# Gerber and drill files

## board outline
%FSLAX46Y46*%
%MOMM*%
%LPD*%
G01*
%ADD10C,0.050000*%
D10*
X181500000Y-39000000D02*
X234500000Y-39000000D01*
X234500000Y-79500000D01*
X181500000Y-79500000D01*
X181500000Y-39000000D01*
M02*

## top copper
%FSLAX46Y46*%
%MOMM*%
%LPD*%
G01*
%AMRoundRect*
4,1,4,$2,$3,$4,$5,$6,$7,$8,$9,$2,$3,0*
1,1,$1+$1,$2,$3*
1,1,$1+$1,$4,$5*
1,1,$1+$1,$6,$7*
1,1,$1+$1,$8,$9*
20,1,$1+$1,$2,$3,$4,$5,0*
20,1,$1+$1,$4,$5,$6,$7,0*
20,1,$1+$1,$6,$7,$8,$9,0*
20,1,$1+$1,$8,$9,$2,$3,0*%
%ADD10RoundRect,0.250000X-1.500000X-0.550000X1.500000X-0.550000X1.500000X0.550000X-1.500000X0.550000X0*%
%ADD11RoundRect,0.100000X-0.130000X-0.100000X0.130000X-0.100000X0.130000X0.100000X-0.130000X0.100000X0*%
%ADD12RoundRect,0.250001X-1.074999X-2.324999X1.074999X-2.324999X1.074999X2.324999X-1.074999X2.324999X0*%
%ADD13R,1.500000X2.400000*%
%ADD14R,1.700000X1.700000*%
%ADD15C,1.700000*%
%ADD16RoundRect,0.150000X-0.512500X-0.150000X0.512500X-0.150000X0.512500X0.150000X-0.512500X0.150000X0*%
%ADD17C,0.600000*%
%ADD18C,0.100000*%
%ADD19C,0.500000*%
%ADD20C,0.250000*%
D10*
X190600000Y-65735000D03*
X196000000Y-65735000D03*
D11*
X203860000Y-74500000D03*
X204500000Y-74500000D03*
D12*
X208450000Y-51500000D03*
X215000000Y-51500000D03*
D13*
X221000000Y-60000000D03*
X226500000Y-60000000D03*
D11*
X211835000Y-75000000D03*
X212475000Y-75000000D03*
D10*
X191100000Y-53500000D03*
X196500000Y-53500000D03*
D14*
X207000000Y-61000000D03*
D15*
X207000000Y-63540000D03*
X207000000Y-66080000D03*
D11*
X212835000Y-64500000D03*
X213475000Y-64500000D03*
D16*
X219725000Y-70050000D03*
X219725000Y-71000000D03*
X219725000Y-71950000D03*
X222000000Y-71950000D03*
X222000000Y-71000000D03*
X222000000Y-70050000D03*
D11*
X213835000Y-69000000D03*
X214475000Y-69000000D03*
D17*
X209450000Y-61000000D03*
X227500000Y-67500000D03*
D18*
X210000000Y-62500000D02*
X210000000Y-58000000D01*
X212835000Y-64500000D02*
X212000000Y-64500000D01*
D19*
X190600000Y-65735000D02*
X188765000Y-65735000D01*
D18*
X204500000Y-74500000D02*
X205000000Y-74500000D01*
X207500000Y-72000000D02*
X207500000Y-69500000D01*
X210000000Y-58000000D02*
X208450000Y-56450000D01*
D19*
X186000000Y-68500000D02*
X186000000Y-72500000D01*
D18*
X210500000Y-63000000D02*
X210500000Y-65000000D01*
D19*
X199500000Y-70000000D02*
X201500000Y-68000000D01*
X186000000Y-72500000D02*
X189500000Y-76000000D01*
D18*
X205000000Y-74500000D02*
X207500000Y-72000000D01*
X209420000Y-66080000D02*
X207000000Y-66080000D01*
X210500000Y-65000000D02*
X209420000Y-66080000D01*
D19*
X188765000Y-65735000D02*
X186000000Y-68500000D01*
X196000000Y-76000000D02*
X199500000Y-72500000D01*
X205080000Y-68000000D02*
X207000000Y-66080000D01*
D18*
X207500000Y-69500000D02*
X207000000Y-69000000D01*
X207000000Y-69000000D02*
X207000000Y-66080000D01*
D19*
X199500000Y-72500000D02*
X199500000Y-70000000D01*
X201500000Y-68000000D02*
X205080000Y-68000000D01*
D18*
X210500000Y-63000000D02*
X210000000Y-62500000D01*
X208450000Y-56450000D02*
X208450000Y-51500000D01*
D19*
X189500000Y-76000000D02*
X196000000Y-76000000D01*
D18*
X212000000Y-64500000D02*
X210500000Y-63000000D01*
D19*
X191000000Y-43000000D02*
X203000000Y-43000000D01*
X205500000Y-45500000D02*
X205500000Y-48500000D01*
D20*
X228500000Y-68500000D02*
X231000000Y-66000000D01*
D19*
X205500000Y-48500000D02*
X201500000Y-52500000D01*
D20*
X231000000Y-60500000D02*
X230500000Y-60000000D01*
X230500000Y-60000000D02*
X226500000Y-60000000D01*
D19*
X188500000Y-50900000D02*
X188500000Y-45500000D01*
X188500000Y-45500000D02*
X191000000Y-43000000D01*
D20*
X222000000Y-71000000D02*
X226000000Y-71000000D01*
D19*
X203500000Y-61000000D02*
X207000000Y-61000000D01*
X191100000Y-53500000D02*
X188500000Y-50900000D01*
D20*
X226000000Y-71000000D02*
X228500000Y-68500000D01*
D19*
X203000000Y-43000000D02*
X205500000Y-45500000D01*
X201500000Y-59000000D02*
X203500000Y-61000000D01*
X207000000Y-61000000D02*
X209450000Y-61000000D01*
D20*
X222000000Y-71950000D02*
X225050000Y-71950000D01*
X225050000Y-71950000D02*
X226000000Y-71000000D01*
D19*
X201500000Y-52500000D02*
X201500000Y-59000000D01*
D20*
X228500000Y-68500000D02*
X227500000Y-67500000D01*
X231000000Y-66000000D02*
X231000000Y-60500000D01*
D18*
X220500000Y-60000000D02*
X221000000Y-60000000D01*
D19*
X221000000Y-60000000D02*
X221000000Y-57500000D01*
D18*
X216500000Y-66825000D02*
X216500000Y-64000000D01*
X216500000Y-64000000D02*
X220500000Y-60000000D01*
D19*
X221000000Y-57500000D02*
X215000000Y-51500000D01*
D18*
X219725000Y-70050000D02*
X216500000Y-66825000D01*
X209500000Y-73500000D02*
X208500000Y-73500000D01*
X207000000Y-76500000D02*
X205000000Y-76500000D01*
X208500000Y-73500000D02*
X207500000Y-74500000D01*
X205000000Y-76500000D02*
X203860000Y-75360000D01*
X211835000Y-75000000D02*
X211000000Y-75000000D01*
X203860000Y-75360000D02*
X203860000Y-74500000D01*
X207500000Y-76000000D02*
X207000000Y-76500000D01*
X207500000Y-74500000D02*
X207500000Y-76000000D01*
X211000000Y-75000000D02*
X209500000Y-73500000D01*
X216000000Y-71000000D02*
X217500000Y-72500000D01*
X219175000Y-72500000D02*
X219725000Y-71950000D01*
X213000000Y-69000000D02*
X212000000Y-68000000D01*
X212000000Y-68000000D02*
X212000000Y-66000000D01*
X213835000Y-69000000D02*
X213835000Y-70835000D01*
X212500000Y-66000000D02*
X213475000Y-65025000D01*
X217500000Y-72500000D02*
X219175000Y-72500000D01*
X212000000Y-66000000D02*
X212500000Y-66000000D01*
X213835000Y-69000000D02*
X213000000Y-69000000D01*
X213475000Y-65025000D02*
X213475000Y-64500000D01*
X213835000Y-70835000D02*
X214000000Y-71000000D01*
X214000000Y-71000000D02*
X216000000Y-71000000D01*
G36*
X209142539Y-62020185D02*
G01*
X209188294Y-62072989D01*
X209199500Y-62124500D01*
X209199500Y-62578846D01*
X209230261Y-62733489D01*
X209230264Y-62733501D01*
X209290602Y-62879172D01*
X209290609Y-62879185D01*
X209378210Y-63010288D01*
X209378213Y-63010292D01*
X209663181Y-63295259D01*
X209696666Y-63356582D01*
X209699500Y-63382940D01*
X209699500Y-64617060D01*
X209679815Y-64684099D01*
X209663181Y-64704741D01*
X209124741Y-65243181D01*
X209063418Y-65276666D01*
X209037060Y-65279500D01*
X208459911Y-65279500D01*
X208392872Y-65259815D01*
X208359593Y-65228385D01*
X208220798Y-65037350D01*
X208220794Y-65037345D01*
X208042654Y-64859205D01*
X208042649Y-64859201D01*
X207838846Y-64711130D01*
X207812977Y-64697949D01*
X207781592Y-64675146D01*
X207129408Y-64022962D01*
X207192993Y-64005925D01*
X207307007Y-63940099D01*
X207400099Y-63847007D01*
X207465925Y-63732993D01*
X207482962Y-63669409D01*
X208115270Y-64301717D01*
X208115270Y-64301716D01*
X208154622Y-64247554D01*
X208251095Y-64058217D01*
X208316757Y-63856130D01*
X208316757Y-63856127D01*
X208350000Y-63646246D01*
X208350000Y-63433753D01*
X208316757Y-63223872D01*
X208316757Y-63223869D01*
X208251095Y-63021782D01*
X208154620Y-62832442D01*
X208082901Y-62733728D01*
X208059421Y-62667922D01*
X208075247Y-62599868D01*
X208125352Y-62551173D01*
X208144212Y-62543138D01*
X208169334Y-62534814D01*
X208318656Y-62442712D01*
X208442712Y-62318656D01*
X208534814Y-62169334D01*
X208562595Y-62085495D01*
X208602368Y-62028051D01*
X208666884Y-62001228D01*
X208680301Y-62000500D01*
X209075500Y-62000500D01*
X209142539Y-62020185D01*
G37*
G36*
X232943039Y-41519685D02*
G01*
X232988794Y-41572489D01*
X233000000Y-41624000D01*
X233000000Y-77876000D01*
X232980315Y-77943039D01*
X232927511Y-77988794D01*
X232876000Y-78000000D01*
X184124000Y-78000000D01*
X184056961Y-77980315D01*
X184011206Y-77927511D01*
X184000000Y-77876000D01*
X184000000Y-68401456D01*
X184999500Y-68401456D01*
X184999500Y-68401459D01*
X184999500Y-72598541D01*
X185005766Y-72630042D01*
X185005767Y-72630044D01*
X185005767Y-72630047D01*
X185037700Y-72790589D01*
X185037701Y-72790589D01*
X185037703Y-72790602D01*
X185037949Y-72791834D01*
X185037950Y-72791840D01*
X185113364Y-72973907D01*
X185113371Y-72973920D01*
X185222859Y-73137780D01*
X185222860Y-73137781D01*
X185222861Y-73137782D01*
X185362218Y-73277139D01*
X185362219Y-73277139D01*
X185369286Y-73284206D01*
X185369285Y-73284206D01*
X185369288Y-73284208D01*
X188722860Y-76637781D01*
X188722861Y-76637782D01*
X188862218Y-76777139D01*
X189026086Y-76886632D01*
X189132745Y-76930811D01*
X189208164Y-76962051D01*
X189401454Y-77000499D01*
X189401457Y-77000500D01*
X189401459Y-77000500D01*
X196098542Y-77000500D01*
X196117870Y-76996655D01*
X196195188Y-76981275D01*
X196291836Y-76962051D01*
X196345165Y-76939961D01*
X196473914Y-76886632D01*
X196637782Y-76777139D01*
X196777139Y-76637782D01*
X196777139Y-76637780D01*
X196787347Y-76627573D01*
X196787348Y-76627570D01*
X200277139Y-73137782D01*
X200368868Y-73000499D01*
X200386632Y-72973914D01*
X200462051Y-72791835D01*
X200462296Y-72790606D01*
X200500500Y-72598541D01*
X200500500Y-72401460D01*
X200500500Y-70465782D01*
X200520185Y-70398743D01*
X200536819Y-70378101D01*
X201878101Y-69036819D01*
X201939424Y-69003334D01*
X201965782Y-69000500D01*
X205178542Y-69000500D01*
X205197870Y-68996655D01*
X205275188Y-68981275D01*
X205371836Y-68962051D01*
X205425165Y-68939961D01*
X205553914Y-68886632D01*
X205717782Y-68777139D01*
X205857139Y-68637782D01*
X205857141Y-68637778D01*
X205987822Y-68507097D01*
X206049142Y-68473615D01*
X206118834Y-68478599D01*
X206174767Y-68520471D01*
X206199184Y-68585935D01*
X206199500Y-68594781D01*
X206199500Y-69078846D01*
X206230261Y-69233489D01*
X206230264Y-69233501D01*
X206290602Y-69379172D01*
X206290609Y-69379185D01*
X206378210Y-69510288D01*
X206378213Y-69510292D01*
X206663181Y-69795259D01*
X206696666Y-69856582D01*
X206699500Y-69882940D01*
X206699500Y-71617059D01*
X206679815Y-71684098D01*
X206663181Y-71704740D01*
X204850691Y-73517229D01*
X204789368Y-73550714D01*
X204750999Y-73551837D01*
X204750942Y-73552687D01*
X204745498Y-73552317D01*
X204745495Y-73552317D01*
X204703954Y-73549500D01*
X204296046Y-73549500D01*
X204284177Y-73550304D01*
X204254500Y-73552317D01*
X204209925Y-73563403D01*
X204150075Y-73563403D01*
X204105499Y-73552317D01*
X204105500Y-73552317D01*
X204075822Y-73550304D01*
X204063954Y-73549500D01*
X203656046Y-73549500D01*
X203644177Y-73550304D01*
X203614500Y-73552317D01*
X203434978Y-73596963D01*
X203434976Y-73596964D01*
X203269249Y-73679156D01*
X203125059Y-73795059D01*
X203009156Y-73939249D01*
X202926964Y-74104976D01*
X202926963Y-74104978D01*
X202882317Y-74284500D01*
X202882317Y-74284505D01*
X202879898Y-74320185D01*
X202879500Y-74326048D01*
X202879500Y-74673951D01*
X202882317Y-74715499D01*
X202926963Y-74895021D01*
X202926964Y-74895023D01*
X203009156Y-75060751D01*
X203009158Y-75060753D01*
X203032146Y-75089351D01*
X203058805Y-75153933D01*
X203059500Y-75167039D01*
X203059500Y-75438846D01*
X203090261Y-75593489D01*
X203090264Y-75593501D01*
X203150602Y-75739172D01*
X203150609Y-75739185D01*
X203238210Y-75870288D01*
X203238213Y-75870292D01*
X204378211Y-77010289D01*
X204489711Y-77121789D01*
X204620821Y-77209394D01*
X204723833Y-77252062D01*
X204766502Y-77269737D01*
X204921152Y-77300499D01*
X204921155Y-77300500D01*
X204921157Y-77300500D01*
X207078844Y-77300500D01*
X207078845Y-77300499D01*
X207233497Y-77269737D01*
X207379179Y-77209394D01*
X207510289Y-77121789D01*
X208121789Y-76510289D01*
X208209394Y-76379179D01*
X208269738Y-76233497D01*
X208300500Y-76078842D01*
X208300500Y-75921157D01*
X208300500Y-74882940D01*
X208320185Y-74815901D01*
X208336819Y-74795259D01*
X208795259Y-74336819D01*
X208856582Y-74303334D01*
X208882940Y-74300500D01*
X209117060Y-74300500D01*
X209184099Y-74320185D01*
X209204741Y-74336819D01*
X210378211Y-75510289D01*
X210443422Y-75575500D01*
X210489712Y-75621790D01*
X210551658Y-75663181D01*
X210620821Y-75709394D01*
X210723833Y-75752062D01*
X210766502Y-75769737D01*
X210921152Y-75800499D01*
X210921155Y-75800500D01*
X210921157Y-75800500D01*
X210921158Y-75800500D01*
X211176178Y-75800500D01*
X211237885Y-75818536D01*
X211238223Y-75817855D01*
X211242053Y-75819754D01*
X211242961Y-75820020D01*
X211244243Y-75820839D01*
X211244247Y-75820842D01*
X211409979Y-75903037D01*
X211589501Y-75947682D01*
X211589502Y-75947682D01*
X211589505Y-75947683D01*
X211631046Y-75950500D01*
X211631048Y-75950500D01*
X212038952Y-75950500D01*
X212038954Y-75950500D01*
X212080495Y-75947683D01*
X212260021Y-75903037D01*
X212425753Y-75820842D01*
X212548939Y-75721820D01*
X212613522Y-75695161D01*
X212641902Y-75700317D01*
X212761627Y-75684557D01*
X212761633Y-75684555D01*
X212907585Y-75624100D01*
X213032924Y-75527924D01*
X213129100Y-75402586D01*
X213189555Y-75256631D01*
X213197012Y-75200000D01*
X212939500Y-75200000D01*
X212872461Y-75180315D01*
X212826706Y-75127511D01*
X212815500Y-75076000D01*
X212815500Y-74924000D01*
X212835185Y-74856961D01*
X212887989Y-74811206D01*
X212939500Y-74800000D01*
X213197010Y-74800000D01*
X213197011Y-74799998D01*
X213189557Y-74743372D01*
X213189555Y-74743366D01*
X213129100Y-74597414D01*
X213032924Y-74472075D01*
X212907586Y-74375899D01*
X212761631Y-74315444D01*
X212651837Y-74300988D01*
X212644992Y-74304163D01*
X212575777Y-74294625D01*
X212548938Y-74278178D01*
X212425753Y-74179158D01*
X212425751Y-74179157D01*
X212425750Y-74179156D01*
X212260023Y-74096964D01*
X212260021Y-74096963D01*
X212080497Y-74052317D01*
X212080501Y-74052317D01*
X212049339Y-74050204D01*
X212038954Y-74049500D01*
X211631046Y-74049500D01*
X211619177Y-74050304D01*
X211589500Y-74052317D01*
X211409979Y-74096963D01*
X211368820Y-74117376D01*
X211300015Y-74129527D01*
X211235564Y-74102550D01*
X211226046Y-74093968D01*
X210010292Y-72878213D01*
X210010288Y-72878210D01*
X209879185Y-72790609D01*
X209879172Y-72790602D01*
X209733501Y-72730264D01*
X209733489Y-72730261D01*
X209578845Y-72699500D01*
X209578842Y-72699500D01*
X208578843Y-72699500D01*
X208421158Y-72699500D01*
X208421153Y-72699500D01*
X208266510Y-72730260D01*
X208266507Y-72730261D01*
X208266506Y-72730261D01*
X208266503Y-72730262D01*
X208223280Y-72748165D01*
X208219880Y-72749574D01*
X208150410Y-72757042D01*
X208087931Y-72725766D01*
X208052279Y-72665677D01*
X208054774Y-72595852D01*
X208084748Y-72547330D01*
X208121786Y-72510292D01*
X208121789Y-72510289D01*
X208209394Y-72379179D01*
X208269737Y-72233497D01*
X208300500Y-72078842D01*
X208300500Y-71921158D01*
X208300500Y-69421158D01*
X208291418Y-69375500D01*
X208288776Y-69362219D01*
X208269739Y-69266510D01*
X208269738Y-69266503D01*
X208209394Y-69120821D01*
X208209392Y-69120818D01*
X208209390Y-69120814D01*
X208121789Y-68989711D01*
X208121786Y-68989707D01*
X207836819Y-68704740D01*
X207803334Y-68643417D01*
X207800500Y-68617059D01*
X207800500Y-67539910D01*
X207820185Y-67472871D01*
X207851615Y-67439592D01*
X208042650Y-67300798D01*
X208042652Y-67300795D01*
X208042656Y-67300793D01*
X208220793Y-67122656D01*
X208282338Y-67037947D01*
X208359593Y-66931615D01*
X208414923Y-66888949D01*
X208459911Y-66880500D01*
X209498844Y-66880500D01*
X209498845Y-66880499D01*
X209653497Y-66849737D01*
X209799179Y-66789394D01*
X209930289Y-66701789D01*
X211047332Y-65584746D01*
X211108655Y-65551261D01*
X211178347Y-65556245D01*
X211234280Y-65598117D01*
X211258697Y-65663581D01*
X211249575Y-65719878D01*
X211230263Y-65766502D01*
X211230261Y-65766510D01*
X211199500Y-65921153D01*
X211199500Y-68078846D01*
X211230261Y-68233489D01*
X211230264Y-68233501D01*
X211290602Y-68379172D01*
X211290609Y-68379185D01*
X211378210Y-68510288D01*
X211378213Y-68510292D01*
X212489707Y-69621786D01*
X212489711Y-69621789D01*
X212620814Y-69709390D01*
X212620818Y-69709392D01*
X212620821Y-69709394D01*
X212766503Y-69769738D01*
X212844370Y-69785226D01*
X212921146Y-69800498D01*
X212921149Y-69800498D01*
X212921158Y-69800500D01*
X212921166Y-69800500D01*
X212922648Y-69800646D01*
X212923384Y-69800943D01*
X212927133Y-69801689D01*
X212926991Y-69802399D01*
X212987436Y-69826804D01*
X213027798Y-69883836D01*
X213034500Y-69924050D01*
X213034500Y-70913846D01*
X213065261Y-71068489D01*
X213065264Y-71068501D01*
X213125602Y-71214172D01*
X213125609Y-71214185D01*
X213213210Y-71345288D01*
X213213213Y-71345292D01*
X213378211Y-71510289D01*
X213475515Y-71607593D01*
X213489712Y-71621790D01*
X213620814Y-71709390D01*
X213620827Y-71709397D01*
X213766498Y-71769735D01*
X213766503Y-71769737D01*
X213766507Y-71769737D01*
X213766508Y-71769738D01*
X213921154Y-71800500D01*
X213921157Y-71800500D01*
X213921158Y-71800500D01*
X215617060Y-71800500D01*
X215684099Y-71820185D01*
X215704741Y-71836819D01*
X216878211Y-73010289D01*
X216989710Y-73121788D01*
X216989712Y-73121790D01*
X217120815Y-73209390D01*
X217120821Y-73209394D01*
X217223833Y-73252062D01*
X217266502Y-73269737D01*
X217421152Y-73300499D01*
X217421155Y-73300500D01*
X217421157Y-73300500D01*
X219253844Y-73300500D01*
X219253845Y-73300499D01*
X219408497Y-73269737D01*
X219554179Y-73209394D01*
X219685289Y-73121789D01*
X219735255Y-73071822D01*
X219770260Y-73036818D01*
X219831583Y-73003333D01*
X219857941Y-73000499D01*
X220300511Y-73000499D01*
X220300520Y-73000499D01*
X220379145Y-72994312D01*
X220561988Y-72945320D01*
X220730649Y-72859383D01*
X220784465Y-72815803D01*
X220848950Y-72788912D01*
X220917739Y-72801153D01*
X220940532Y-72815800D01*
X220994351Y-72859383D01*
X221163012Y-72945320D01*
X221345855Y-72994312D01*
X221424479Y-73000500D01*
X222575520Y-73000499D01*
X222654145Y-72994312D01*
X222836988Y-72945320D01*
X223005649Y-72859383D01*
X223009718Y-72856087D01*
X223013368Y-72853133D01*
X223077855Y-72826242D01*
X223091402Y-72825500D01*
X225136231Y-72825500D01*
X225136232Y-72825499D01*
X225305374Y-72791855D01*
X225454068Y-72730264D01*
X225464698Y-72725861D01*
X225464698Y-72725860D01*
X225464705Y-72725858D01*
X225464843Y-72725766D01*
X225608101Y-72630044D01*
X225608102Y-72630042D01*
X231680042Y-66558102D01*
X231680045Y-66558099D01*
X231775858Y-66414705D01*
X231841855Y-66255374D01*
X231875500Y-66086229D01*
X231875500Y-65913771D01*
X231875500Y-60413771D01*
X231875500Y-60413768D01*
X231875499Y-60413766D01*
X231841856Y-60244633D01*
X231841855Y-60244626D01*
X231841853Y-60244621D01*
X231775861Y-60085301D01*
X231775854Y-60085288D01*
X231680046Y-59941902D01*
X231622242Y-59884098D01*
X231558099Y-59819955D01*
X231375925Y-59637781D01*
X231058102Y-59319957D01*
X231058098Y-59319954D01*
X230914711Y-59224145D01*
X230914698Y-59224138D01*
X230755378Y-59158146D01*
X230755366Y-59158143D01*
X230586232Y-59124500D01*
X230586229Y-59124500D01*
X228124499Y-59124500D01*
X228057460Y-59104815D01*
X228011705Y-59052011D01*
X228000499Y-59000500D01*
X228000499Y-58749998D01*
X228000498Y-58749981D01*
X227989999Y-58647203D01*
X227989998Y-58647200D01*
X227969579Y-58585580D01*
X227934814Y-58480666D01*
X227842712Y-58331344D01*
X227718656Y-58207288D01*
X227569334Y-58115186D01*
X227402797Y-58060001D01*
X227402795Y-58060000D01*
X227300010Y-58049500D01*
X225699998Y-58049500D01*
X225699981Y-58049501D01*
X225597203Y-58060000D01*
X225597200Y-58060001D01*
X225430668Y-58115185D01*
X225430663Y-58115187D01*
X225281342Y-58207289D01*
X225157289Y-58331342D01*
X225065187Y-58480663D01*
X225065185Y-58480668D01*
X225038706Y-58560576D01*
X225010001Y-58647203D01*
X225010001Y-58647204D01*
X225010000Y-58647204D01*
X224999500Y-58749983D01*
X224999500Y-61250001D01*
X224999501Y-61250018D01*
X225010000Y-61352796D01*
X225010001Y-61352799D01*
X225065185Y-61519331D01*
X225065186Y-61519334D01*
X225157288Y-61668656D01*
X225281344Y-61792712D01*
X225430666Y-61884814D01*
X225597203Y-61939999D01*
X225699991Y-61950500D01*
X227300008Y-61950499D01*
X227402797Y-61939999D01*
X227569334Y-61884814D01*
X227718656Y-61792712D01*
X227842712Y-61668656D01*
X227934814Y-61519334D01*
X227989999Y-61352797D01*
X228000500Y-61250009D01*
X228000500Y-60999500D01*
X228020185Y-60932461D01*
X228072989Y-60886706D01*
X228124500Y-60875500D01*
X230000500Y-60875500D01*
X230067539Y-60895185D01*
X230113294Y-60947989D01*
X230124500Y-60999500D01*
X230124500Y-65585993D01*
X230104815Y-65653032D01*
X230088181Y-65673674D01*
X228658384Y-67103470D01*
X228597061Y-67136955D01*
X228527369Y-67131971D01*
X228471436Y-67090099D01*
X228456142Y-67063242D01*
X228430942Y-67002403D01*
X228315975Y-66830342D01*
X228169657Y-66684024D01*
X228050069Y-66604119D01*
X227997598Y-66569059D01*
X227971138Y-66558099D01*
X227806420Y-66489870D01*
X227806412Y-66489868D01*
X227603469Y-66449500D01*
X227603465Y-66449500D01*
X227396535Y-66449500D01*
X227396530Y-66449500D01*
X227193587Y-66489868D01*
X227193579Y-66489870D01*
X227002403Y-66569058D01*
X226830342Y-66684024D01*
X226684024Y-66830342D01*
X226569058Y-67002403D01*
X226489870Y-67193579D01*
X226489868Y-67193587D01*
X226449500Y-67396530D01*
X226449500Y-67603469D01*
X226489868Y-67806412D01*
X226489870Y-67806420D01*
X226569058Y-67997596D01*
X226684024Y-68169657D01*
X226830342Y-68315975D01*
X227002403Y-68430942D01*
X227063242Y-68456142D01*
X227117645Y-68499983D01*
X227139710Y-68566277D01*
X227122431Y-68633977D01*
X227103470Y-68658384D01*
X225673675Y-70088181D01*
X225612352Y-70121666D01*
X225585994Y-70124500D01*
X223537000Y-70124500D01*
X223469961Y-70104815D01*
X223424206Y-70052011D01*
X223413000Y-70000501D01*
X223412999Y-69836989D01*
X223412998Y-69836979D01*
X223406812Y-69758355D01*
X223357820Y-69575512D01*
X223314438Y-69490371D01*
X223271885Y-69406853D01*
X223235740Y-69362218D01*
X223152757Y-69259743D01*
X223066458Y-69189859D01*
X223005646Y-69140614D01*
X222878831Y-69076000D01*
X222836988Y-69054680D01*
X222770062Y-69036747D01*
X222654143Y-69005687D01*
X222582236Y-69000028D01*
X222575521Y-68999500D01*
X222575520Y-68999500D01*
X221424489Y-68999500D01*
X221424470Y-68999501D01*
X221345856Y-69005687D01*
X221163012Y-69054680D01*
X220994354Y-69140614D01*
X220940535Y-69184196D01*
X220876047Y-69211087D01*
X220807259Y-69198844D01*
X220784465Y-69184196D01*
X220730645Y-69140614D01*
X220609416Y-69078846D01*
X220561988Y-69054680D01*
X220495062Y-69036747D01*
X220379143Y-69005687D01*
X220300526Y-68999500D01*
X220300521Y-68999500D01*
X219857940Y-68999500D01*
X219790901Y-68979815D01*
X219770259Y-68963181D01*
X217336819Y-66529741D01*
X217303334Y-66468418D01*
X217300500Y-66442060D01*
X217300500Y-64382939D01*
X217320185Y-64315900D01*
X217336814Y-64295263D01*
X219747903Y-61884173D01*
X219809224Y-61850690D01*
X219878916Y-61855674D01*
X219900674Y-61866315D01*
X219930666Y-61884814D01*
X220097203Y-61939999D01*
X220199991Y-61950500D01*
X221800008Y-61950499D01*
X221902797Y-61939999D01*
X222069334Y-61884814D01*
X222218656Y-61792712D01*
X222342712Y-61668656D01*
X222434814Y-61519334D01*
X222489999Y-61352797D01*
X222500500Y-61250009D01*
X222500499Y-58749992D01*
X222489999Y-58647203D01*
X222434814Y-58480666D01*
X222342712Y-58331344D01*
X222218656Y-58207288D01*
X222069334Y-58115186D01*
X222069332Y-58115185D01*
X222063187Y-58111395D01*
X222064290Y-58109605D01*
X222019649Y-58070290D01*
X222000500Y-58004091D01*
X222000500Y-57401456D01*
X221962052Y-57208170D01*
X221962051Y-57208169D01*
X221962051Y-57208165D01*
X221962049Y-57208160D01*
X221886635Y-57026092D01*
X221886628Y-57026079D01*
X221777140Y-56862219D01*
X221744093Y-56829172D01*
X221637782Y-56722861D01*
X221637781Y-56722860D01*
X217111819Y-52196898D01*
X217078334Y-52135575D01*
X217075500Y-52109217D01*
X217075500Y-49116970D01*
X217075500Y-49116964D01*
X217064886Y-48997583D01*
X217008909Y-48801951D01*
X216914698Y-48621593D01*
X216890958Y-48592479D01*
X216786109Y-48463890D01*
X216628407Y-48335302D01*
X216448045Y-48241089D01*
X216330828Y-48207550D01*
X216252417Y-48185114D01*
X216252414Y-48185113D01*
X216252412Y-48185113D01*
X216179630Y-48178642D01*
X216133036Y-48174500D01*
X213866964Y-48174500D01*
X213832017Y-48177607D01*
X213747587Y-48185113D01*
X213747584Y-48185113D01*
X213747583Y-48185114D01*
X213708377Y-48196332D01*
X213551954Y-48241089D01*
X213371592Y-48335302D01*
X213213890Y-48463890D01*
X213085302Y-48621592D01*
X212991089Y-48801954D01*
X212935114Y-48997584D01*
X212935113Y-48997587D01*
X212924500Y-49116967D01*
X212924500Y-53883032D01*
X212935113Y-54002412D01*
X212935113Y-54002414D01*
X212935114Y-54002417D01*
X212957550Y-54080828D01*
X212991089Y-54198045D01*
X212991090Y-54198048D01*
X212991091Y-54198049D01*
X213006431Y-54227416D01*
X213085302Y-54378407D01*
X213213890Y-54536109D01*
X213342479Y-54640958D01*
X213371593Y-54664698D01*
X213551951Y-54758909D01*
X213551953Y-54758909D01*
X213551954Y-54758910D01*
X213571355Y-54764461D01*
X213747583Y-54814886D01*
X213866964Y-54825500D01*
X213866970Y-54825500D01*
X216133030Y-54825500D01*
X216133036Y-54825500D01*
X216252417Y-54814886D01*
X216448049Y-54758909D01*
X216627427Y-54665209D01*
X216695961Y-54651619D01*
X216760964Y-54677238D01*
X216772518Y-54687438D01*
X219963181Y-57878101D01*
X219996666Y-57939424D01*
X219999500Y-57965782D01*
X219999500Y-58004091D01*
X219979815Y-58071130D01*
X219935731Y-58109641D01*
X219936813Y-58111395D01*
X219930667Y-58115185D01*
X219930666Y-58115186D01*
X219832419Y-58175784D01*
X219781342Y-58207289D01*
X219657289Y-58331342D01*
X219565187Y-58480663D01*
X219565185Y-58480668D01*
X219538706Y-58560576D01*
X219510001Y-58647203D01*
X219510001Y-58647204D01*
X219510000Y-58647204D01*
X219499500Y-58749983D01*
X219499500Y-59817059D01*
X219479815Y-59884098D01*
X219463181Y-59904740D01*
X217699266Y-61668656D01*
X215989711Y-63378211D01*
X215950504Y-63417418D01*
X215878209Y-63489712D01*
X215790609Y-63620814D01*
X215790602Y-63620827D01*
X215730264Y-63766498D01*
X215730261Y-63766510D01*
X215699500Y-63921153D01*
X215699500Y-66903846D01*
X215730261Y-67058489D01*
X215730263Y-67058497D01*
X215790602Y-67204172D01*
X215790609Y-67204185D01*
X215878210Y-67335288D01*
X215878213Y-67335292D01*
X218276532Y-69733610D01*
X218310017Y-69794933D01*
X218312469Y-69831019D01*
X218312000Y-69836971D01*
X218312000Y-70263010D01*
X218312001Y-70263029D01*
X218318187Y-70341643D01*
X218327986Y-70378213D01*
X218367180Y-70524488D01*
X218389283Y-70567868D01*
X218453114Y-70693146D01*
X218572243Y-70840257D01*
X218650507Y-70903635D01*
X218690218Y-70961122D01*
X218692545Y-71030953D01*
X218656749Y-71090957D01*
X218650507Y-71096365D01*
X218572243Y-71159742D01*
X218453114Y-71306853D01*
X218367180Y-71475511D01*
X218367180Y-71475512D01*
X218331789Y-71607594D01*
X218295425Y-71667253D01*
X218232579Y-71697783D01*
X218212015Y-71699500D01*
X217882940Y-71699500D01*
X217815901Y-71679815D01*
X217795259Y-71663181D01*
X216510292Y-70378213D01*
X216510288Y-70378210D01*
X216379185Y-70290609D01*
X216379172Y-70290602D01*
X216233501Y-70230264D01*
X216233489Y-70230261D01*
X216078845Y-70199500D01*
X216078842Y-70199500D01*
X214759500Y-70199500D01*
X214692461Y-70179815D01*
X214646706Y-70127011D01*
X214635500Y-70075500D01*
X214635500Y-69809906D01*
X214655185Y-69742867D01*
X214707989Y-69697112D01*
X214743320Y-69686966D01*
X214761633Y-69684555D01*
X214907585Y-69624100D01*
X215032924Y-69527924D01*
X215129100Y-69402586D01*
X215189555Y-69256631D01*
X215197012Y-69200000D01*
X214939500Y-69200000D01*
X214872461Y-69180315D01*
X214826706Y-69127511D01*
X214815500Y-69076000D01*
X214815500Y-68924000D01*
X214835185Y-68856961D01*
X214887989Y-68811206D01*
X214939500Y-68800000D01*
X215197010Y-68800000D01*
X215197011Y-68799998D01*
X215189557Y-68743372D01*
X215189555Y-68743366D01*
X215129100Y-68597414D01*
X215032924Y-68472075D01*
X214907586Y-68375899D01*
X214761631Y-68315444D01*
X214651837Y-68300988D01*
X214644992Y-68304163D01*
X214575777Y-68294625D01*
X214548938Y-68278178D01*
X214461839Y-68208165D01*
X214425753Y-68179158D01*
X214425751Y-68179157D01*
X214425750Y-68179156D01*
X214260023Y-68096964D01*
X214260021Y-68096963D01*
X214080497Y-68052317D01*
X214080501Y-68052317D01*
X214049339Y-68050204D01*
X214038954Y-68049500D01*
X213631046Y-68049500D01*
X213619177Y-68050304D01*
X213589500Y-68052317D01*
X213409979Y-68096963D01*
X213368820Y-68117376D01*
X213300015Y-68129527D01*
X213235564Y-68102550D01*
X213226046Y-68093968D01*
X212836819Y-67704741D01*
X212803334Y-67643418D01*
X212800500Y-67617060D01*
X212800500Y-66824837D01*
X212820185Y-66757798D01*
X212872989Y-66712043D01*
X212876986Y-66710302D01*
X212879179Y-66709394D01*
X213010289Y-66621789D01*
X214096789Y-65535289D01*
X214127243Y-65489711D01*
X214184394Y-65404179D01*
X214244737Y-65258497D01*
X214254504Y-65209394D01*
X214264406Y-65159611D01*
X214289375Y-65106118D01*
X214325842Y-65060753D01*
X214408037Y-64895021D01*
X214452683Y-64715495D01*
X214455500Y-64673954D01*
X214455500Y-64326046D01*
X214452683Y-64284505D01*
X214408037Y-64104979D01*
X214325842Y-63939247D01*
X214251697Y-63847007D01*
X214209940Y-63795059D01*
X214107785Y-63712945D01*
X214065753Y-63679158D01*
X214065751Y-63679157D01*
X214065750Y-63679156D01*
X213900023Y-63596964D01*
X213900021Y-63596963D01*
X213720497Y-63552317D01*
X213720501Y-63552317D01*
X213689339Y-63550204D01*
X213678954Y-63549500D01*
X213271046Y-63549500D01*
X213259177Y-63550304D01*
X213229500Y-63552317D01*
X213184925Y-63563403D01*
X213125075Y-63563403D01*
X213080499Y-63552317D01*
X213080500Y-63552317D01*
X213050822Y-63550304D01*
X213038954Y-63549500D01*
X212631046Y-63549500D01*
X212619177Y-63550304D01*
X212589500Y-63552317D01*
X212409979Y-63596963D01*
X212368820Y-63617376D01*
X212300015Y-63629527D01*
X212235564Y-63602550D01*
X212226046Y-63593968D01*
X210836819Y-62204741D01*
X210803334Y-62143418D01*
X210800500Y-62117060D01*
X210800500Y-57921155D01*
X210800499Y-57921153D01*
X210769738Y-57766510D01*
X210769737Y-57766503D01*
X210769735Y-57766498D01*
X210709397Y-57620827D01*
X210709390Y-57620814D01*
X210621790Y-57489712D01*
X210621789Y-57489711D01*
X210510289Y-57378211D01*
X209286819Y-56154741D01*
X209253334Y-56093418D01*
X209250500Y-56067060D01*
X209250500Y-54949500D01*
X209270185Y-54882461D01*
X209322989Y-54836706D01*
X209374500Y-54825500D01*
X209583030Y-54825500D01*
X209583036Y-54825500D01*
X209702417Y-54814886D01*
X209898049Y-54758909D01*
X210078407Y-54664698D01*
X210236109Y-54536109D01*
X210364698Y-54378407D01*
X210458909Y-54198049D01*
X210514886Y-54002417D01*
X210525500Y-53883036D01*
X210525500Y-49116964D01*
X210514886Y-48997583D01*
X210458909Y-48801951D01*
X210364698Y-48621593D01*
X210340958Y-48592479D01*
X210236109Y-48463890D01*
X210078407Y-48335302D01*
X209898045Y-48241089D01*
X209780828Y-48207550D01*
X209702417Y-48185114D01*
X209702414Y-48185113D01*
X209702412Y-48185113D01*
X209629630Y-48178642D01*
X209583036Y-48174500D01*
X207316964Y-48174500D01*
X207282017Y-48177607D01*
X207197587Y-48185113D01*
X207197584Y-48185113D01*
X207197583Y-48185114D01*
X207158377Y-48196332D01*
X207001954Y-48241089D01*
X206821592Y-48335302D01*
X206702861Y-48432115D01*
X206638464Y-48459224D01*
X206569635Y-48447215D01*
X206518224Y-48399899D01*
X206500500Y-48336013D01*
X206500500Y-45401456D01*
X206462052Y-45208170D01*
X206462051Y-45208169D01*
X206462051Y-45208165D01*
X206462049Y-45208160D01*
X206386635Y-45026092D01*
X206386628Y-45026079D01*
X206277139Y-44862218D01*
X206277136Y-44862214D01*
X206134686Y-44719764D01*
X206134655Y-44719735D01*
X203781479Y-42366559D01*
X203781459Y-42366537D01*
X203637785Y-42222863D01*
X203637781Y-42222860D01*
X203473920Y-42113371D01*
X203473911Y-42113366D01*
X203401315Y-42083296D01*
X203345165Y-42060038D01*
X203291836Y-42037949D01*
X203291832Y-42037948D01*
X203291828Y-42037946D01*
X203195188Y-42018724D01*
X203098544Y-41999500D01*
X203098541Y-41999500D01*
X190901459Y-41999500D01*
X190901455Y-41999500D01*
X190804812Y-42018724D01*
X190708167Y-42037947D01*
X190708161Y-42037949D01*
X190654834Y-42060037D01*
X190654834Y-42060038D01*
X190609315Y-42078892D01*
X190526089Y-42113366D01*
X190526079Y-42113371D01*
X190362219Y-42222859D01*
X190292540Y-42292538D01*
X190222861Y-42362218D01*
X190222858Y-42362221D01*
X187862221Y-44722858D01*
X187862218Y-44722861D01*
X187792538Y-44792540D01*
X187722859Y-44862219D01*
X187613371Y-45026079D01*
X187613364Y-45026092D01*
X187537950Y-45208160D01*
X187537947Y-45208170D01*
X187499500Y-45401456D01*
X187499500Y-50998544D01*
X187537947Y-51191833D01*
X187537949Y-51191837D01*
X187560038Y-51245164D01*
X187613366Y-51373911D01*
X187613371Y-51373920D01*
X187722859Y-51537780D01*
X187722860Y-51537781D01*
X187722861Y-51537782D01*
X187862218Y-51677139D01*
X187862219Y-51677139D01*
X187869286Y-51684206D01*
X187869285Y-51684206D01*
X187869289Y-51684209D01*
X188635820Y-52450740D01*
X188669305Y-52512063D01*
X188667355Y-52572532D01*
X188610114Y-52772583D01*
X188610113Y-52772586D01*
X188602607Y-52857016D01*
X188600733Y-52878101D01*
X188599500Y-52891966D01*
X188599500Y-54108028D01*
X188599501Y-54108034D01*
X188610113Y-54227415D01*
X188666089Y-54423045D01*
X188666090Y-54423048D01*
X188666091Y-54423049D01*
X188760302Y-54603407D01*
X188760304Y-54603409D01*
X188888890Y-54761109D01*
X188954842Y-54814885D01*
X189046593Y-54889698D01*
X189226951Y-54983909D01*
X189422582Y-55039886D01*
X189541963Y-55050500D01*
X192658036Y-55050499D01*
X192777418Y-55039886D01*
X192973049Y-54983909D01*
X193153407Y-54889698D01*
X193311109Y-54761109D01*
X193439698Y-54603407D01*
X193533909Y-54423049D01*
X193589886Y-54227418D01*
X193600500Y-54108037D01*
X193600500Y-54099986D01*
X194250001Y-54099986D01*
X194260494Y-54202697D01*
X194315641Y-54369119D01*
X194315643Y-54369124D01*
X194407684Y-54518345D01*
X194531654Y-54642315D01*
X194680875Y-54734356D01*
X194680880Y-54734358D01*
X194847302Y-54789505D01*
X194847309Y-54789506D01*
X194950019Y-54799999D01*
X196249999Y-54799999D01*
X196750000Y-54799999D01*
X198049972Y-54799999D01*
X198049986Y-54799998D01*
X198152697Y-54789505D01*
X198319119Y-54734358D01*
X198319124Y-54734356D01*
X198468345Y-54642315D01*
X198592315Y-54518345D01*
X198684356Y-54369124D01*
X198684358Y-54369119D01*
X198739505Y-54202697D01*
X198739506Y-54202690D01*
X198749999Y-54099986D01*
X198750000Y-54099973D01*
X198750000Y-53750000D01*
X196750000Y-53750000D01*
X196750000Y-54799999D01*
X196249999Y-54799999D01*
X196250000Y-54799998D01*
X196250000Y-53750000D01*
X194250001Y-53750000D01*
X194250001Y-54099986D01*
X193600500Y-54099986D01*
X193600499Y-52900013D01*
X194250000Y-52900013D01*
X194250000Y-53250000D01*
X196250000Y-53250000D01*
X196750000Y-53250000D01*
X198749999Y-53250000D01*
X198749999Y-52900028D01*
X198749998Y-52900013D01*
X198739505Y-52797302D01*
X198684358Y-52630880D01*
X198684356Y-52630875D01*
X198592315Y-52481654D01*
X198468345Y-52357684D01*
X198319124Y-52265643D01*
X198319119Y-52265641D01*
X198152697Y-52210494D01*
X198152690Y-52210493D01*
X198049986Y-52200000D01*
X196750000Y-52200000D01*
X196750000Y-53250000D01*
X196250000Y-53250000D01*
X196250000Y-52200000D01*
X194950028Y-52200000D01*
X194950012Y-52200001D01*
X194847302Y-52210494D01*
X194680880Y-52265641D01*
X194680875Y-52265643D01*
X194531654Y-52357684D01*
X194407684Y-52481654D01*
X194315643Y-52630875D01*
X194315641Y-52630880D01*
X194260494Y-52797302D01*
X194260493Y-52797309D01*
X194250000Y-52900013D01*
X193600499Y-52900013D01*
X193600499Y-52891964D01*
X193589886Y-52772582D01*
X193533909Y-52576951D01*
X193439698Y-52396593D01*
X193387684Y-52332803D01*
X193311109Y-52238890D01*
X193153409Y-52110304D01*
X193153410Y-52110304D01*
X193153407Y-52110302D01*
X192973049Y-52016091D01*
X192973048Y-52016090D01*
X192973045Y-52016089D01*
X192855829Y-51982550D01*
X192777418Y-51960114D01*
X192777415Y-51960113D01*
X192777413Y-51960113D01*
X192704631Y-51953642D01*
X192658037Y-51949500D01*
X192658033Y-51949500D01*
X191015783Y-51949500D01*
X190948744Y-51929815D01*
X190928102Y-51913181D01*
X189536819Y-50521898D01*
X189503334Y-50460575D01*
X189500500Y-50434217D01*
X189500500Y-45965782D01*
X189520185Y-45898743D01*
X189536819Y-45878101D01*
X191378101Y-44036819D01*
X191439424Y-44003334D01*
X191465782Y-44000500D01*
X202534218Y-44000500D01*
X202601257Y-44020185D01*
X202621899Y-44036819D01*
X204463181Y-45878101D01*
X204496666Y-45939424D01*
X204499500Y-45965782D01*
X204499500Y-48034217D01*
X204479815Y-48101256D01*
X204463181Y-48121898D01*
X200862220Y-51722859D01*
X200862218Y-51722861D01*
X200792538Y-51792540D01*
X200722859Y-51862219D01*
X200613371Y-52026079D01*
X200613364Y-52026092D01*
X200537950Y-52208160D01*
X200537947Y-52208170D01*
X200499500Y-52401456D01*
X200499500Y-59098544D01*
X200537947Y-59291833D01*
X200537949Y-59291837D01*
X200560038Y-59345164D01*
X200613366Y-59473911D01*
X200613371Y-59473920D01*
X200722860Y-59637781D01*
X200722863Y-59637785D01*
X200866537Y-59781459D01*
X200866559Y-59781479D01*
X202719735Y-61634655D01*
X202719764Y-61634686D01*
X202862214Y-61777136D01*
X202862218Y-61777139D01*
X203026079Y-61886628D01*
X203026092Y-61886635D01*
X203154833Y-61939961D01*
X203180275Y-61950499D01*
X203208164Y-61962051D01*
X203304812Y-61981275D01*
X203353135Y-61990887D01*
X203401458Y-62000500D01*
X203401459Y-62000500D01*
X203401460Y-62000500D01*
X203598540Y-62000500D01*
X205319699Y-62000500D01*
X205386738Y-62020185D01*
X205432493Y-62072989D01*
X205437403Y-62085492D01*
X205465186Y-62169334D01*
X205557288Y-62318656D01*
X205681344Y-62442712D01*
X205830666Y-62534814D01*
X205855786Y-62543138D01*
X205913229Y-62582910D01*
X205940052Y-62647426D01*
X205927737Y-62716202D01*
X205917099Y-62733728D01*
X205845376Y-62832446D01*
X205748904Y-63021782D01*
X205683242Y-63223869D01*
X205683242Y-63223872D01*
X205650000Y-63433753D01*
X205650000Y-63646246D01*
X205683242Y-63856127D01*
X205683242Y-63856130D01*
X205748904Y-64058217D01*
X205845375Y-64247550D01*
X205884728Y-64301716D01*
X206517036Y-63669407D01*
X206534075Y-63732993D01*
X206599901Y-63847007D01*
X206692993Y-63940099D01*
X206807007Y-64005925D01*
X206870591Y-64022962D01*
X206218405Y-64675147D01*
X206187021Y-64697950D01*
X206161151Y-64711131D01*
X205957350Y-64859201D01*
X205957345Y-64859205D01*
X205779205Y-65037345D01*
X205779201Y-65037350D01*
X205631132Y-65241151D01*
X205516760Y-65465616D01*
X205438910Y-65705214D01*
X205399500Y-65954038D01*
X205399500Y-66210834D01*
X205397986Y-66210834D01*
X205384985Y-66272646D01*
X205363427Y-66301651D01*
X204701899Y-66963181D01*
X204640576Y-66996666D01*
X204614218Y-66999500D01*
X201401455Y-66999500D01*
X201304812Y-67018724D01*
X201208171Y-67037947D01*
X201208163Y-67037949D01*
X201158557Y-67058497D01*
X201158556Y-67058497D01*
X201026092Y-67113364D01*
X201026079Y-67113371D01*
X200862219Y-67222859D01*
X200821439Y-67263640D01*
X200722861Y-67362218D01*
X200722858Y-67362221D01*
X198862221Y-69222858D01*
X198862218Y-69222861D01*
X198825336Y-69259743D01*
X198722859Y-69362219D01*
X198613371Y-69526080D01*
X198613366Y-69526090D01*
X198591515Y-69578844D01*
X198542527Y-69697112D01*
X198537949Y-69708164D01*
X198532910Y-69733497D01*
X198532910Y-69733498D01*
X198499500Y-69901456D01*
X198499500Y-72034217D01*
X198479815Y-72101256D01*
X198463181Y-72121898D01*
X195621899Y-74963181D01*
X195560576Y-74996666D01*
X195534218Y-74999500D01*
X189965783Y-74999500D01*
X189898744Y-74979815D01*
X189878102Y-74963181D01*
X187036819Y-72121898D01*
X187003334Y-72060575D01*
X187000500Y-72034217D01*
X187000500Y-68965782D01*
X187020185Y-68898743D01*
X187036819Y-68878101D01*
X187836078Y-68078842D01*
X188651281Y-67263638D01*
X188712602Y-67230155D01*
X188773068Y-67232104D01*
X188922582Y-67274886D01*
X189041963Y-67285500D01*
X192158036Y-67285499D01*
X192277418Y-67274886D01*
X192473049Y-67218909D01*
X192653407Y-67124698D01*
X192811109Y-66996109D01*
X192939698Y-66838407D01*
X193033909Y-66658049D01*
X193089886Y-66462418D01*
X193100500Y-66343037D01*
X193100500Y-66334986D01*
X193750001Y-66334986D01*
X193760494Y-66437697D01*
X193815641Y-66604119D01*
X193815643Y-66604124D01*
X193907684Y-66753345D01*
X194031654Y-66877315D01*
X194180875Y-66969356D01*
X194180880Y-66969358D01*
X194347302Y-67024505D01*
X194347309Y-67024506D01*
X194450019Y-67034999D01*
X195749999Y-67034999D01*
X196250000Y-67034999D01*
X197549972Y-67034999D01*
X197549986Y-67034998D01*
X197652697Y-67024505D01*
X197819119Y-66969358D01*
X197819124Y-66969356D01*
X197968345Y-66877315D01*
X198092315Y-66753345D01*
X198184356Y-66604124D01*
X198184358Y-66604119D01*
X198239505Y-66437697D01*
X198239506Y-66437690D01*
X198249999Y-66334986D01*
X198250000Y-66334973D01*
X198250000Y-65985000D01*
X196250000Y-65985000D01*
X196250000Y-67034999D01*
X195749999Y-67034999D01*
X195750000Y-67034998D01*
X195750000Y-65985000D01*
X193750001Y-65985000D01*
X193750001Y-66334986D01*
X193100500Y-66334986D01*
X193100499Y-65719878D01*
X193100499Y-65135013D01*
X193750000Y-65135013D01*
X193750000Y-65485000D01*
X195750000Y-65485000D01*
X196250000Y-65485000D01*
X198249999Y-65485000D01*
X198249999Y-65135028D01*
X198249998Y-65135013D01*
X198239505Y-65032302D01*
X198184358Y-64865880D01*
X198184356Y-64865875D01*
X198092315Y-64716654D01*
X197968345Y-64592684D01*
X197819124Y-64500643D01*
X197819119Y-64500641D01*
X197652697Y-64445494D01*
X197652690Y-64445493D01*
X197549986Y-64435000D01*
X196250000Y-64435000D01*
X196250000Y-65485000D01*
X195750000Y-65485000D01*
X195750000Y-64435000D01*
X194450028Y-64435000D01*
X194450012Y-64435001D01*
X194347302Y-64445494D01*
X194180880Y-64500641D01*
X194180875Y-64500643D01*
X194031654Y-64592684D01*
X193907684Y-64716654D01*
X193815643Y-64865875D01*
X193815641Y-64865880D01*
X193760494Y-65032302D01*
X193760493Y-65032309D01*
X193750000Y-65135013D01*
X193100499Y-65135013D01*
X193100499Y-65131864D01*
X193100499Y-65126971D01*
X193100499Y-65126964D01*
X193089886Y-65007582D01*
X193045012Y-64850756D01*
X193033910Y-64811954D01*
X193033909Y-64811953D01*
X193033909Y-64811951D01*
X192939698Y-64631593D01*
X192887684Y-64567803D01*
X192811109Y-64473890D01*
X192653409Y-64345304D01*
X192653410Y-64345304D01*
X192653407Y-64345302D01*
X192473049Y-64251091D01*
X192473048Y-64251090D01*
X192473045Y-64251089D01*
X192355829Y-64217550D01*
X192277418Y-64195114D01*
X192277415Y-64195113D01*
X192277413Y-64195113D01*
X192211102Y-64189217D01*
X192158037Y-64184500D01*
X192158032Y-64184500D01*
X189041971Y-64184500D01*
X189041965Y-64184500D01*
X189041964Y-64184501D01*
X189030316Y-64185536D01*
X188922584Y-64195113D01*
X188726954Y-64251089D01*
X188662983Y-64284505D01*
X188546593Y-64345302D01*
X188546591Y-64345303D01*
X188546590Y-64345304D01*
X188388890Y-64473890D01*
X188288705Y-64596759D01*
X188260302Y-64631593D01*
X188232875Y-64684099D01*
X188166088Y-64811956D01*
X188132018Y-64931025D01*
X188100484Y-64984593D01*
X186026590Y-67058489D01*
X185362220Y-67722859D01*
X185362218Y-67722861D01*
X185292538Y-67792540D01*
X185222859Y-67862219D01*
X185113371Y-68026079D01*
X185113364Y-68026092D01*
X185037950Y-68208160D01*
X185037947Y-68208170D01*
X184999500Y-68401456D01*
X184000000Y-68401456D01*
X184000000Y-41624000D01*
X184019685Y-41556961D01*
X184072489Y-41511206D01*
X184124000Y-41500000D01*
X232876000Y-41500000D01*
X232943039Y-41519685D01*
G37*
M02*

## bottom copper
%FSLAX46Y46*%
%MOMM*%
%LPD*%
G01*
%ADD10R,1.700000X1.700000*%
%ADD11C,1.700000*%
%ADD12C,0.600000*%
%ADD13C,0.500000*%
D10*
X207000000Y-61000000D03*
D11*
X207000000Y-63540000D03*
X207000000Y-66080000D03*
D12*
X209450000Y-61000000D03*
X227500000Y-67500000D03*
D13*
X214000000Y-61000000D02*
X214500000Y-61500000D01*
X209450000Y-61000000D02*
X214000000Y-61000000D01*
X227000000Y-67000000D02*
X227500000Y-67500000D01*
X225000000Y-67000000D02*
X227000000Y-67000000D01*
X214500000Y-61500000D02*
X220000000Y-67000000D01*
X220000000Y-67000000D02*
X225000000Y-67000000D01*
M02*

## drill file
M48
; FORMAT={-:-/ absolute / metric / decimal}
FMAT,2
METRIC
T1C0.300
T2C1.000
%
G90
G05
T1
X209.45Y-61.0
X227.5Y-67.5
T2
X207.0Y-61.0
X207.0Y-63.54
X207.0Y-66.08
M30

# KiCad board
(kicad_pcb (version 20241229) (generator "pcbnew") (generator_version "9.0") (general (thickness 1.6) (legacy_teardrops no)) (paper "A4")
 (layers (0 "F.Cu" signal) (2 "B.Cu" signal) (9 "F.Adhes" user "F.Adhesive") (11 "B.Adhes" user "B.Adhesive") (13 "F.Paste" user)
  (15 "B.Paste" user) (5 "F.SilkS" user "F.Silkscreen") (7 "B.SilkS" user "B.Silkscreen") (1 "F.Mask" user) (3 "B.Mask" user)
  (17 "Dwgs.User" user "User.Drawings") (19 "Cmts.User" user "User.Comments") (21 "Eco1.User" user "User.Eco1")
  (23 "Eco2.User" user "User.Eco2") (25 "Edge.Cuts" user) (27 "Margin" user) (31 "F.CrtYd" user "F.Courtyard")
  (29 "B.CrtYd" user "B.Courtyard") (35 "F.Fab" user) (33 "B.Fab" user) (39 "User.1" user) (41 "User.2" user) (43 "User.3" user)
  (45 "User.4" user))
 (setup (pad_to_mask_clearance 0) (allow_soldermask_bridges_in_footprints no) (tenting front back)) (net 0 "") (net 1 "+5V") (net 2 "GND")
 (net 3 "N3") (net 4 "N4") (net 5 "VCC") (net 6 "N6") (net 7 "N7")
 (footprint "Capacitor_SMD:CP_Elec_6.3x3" (layer "F.Cu") (at 193.3 65.735)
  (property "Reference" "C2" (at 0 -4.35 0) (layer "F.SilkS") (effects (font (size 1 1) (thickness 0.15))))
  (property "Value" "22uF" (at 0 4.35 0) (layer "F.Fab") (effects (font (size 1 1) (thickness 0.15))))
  (pad "1" smd roundrect (at -2.7 0) (size 3.5 1.6) (layers "F.Cu" "F.Mask" "F.Paste") (roundrect_rratio 0.15625) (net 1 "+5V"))
  (pad "2" smd roundrect (at 2.7 0) (size 3.5 1.6) (layers "F.Cu" "F.Mask" "F.Paste") (roundrect_rratio 0.15625) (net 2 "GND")))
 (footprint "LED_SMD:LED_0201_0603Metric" (layer "F.Cu") (at 204.18 74.5)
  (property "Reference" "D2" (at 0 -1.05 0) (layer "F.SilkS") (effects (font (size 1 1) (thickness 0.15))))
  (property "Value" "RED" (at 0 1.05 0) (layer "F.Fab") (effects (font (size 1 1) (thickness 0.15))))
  (pad "" smd roundrect (at -0.345 0) (size 0.318 0.36) (layers "F.Paste") (roundrect_rratio 0.25))
  (pad "" smd roundrect (at 0.345 0) (size 0.318 0.36) (layers "F.Paste") (roundrect_rratio 0.25))
  (pad "1" smd roundrect (at -0.32 0) (size 0.46 0.4) (layers "F.Cu" "F.Mask") (roundrect_rratio 0.25) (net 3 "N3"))
  (pad "2" smd roundrect (at 0.32 0) (size 0.46 0.4) (layers "F.Cu" "F.Mask") (roundrect_rratio 0.25) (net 1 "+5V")))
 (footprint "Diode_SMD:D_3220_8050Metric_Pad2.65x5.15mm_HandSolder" (layer "F.Cu") (at 211.725 51.5)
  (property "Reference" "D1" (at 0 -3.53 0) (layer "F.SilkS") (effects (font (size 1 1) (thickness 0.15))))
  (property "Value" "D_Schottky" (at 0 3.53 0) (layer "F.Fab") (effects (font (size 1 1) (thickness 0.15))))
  (pad "1" smd roundrect (at -3.275 0) (size 2.65 5.15) (layers "F.Cu" "F.Mask" "F.Paste") (roundrect_rratio 0.09434) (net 1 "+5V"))
  (pad "2" smd roundrect (at 3.275 0) (size 2.65 5.15) (layers "F.Cu" "F.Mask" "F.Paste") (roundrect_rratio 0.09434) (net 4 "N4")))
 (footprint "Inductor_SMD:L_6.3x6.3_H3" (layer "F.Cu") (at 223.75 60)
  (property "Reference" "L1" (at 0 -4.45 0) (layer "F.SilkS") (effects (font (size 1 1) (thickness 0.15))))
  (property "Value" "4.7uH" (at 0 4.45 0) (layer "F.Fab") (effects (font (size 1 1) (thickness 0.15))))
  (pad "1" smd rect (at -2.75 0) (size 1.5 2.4) (layers "F.Cu" "F.Mask" "F.Paste") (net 4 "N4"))
  (pad "2" smd rect (at 2.75 0) (size 1.5 2.4) (layers "F.Cu" "F.Mask" "F.Paste") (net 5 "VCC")))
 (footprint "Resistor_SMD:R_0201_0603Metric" (layer "F.Cu") (at 212.155 75)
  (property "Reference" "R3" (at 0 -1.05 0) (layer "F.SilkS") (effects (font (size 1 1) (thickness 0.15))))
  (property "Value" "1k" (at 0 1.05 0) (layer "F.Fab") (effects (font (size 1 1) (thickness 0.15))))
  (pad "" smd roundrect (at -0.345 0) (size 0.318 0.36) (layers "F.Paste") (roundrect_rratio 0.25))
  (pad "" smd roundrect (at 0.345 0) (size 0.318 0.36) (layers "F.Paste") (roundrect_rratio 0.25))
  (pad "1" smd roundrect (at -0.32 0) (size 0.46 0.4) (layers "F.Cu" "F.Mask") (roundrect_rratio 0.25) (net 3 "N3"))
  (pad "2" smd roundrect (at 0.32 0) (size 0.46 0.4) (layers "F.Cu" "F.Mask") (roundrect_rratio 0.25) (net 2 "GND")))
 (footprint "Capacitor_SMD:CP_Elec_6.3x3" (layer "F.Cu") (at 193.8 53.5)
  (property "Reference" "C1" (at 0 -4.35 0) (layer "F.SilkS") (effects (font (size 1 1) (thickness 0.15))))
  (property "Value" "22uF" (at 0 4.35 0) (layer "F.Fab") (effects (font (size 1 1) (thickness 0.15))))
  (pad "1" smd roundrect (at -2.7 0) (size 3.5 1.6) (layers "F.Cu" "F.Mask" "F.Paste") (roundrect_rratio 0.15625) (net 5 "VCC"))
  (pad "2" smd roundrect (at 2.7 0) (size 3.5 1.6) (layers "F.Cu" "F.Mask" "F.Paste") (roundrect_rratio 0.15625) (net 2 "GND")))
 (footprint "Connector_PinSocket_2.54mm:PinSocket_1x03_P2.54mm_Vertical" (layer "F.Cu") (at 207 61)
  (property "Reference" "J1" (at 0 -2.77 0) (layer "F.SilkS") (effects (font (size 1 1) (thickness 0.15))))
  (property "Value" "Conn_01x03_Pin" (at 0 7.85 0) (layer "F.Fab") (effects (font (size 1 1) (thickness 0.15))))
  (pad "1" thru_hole rect (at 0 0) (size 1.7 1.7) (drill 1) (layers "*.Cu" "*.Mask") (remove_unused_layers no) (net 5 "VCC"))
  (pad "2" thru_hole circle (at 0 2.54) (size 1.7 1.7) (drill 1) (layers "*.Cu" "*.Mask") (remove_unused_layers no) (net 2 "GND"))
  (pad "3" thru_hole circle (at 0 5.08) (size 1.7 1.7) (drill 1) (layers "*.Cu" "*.Mask") (remove_unused_layers no) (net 1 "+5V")))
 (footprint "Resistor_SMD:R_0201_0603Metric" (layer "F.Cu") (at 213.155 64.5)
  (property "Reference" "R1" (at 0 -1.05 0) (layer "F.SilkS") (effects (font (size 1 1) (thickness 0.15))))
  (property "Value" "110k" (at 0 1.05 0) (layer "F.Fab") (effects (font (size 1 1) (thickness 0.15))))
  (pad "" smd roundrect (at -0.345 0) (size 0.318 0.36) (layers "F.Paste") (roundrect_rratio 0.25))
  (pad "" smd roundrect (at 0.345 0) (size 0.318 0.36) (layers "F.Paste") (roundrect_rratio 0.25))
  (pad "1" smd roundrect (at -0.32 0) (size 0.46 0.4) (layers "F.Cu" "F.Mask") (roundrect_rratio 0.25) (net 1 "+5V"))
  (pad "2" smd roundrect (at 0.32 0) (size 0.46 0.4) (layers "F.Cu" "F.Mask") (roundrect_rratio 0.25) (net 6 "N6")))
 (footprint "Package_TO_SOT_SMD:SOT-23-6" (layer "F.Cu") (at 220.8625 71)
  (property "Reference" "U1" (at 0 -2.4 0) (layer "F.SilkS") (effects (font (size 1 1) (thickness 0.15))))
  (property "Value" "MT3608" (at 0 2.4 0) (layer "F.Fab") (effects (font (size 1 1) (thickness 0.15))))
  (pad "1" smd roundrect (at -1.1375 -0.95) (size 1.325 0.6) (layers "F.Cu" "F.Mask" "F.Paste") (roundrect_rratio 0.25) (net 4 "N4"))
  (pad "2" smd roundrect (at -1.1375 0) (size 1.325 0.6) (layers "F.Cu" "F.Mask" "F.Paste") (roundrect_rratio 0.25) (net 2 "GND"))
  (pad "3" smd roundrect (at -1.1375 0.95) (size 1.325 0.6) (layers "F.Cu" "F.Mask" "F.Paste") (roundrect_rratio 0.25) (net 6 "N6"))
  (pad "4" smd roundrect (at 1.1375 0.95) (size 1.325 0.6) (layers "F.Cu" "F.Mask" "F.Paste") (roundrect_rratio 0.25) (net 5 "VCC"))
  (pad "5" smd roundrect (at 1.1375 0) (size 1.325 0.6) (layers "F.Cu" "F.Mask" "F.Paste") (roundrect_rratio 0.25) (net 5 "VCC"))
  (pad "6" smd roundrect (at 1.1375 -0.95) (size 1.325 0.6) (layers "F.Cu" "F.Mask" "F.Paste") (roundrect_rratio 0.25) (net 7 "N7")))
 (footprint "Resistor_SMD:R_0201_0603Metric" (layer "F.Cu") (at 214.155 69)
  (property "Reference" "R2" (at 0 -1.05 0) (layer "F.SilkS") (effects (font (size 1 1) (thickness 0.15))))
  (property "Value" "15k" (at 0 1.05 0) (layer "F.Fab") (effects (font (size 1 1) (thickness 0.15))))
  (pad "" smd roundrect (at -0.345 0) (size 0.318 0.36) (layers "F.Paste") (roundrect_rratio 0.25))
  (pad "" smd roundrect (at 0.345 0) (size 0.318 0.36) (layers "F.Paste") (roundrect_rratio 0.25))
  (pad "1" smd roundrect (at -0.32 0) (size 0.46 0.4) (layers "F.Cu" "F.Mask") (roundrect_rratio 0.25) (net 6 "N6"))
  (pad "2" smd roundrect (at 0.32 0) (size 0.46 0.4) (layers "F.Cu" "F.Mask") (roundrect_rratio 0.25) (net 2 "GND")))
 (gr_rect (start 181.5 39) (end 234.5 79.5) (stroke (width 0.05) (type default)) (fill no) (layer "Edge.Cuts"))
 (segment (start 210 62.5) (end 210 58) (width 0.1) (layer "F.Cu") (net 1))
 (segment (start 212.835 64.5) (end 212 64.5) (width 0.1) (layer "F.Cu") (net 1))
 (segment (start 190.6 65.735) (end 188.765 65.735) (width 0.5) (layer "F.Cu") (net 1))
 (segment (start 204.5 74.5) (end 205 74.5) (width 0.1) (layer "F.Cu") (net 1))
 (segment (start 207.5 72) (end 207.5 69.5) (width 0.1) (layer "F.Cu") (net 1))
 (segment (start 210 58) (end 208.45 56.45) (width 0.1) (layer "F.Cu") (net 1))
 (segment (start 186 68.5) (end 186 72.5) (width 0.5) (layer "F.Cu") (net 1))
 (segment (start 210.5 63) (end 210.5 65) (width 0.1) (layer "F.Cu") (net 1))
 (segment (start 199.5 70) (end 201.5 68) (width 0.5) (layer "F.Cu") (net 1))
 (segment (start 186 72.5) (end 189.5 76) (width 0.5) (layer "F.Cu") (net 1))
 (segment (start 205 74.5) (end 207.5 72) (width 0.1) (layer "F.Cu") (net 1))
 (segment (start 209.42 66.08) (end 207 66.08) (width 0.1) (layer "F.Cu") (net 1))
 (segment (start 210.5 65) (end 209.42 66.08) (width 0.1) (layer "F.Cu") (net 1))
 (segment (start 188.765 65.735) (end 186 68.5) (width 0.5) (layer "F.Cu") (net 1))
 (segment (start 196 76) (end 199.5 72.5) (width 0.5) (layer "F.Cu") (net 1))
 (segment (start 205.08 68) (end 207 66.08) (width 0.5) (layer "F.Cu") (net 1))
 (segment (start 207.5 69.5) (end 207 69) (width 0.1) (layer "F.Cu") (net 1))
 (segment (start 207 69) (end 207 66.08) (width 0.1) (layer "F.Cu") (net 1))
 (segment (start 199.5 72.5) (end 199.5 70) (width 0.5) (layer "F.Cu") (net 1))
 (segment (start 201.5 68) (end 205.08 68) (width 0.5) (layer "F.Cu") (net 1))
 (segment (start 210.5 63) (end 210 62.5) (width 0.1) (layer "F.Cu") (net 1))
 (segment (start 208.45 56.45) (end 208.45 51.5) (width 0.1) (layer "F.Cu") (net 1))
 (segment (start 189.5 76) (end 196 76) (width 0.5) (layer "F.Cu") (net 1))
 (segment (start 212 64.5) (end 210.5 63) (width 0.1) (layer "F.Cu") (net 1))
 (segment (start 191 43) (end 203 43) (width 0.5) (layer "F.Cu") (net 5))
 (segment (start 205.5 45.5) (end 205.5 48.5) (width 0.5) (layer "F.Cu") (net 5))
 (segment (start 228.5 68.5) (end 231 66) (width 0.25) (layer "F.Cu") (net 5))
 (segment (start 205.5 48.5) (end 201.5 52.5) (width 0.5) (layer "F.Cu") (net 5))
 (segment (start 231 60.5) (end 230.5 60) (width 0.25) (layer "F.Cu") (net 5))
 (segment (start 230.5 60) (end 226.5 60) (width 0.25) (layer "F.Cu") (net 5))
 (segment (start 188.5 50.9) (end 188.5 45.5) (width 0.5) (layer "F.Cu") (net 5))
 (segment (start 188.5 45.5) (end 191 43) (width 0.5) (layer "F.Cu") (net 5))
 (segment (start 222 71) (end 226 71) (width 0.25) (layer "F.Cu") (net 5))
 (segment (start 203.5 61) (end 207 61) (width 0.5) (layer "F.Cu") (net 5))
 (segment (start 191.1 53.5) (end 188.5 50.9) (width 0.5) (layer "F.Cu") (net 5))
 (segment (start 226 71) (end 228.5 68.5) (width 0.25) (layer "F.Cu") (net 5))
 (segment (start 203 43) (end 205.5 45.5) (width 0.5) (layer "F.Cu") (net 5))
 (segment (start 201.5 59) (end 203.5 61) (width 0.5) (layer "F.Cu") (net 5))
 (segment (start 207 61) (end 209.45 61) (width 0.5) (layer "F.Cu") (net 5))
 (segment (start 222 71.95) (end 225.05 71.95) (width 0.25) (layer "F.Cu") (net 5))
 (segment (start 225.05 71.95) (end 226 71) (width 0.25) (layer "F.Cu") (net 5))
 (segment (start 201.5 52.5) (end 201.5 59) (width 0.5) (layer "F.Cu") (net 5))
 (segment (start 228.5 68.5) (end 227.5 67.5) (width 0.25) (layer "F.Cu") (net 5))
 (segment (start 231 66) (end 231 60.5) (width 0.25) (layer "F.Cu") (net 5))
 (via (at 209.45 61) (size 0.6) (drill 0.3) (layers "F.Cu" "B.Cu") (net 5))
 (via blind (at 227.5 67.5) (size 0.6) (drill 0.3) (layers "F.Cu" "B.Cu") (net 5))
 (segment (start 214 61) (end 214.5 61.5) (width 0.5) (layer "B.Cu") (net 5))
 (segment (start 209.45 61) (end 214 61) (width 0.5) (layer "B.Cu") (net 5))
 (segment (start 227 67) (end 227.5 67.5) (width 0.5) (layer "B.Cu") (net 5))
 (segment (start 225 67) (end 227 67) (width 0.5) (layer "B.Cu") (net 5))
 (segment (start 214.5 61.5) (end 220 67) (width 0.5) (layer "B.Cu") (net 5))
 (segment (start 220 67) (end 225 67) (width 0.5) (layer "B.Cu") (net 5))
 (segment (start 220.5 60) (end 221 60) (width 0.1) (layer "F.Cu") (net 4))
 (segment (start 221 60) (end 221 57.5) (width 0.5) (layer "F.Cu") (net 4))
 (segment (start 216.5 66.825) (end 216.5 64) (width 0.1) (layer "F.Cu") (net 4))
 (segment (start 216.5 64) (end 220.5 60) (width 0.1) (layer "F.Cu") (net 4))
 (segment (start 221 57.5) (end 215 51.5) (width 0.5) (layer "F.Cu") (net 4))
 (segment (start 219.725 70.05) (end 216.5 66.825) (width 0.1) (layer "F.Cu") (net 4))
 (segment (start 209.5 73.5) (end 208.5 73.5) (width 0.1) (layer "F.Cu") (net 3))
 (segment (start 207 76.5) (end 205 76.5) (width 0.1) (layer "F.Cu") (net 3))
 (segment (start 208.5 73.5) (end 207.5 74.5) (width 0.1) (layer "F.Cu") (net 3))
 (segment (start 205 76.5) (end 203.86 75.36) (width 0.1) (layer "F.Cu") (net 3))
 (segment (start 211.835 75) (end 211 75) (width 0.1) (layer "F.Cu") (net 3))
 (segment (start 203.86 75.36) (end 203.86 74.5) (width 0.1) (layer "F.Cu") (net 3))
 (segment (start 207.5 76) (end 207 76.5) (width 0.1) (layer "F.Cu") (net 3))
 (segment (start 207.5 74.5) (end 207.5 76) (width 0.1) (layer "F.Cu") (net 3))
 (segment (start 211 75) (end 209.5 73.5) (width 0.1) (layer "F.Cu") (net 3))
 (segment (start 216 71) (end 217.5 72.5) (width 0.1) (layer "F.Cu") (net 6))
 (segment (start 219.175 72.5) (end 219.725 71.95) (width 0.1) (layer "F.Cu") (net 6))
 (segment (start 213 69) (end 212 68) (width 0.1) (layer "F.Cu") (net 6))
 (segment (start 212 68) (end 212 66) (width 0.1) (layer "F.Cu") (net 6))
 (segment (start 213.835 69) (end 213.835 70.835) (width 0.1) (layer "F.Cu") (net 6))
 (segment (start 212.5 66) (end 213.475 65.025) (width 0.1) (layer "F.Cu") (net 6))
 (segment (start 217.5 72.5) (end 219.175 72.5) (width 0.1) (layer "F.Cu") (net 6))
 (segment (start 212 66) (end 212.5 66) (width 0.1) (layer "F.Cu") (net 6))
 (segment (start 213.835 69) (end 213 69) (width 0.1) (layer "F.Cu") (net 6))
 (segment (start 213.475 65.025) (end 213.475 64.5) (width 0.1) (layer "F.Cu") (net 6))
 (segment (start 213.835 70.835) (end 214 71) (width 0.1) (layer "F.Cu") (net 6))
 (segment (start 214 71) (end 216 71) (width 0.1) (layer "F.Cu") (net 6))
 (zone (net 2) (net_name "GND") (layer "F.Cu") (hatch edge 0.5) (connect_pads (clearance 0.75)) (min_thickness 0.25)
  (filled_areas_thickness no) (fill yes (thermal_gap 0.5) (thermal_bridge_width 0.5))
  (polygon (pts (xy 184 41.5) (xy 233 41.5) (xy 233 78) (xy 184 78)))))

